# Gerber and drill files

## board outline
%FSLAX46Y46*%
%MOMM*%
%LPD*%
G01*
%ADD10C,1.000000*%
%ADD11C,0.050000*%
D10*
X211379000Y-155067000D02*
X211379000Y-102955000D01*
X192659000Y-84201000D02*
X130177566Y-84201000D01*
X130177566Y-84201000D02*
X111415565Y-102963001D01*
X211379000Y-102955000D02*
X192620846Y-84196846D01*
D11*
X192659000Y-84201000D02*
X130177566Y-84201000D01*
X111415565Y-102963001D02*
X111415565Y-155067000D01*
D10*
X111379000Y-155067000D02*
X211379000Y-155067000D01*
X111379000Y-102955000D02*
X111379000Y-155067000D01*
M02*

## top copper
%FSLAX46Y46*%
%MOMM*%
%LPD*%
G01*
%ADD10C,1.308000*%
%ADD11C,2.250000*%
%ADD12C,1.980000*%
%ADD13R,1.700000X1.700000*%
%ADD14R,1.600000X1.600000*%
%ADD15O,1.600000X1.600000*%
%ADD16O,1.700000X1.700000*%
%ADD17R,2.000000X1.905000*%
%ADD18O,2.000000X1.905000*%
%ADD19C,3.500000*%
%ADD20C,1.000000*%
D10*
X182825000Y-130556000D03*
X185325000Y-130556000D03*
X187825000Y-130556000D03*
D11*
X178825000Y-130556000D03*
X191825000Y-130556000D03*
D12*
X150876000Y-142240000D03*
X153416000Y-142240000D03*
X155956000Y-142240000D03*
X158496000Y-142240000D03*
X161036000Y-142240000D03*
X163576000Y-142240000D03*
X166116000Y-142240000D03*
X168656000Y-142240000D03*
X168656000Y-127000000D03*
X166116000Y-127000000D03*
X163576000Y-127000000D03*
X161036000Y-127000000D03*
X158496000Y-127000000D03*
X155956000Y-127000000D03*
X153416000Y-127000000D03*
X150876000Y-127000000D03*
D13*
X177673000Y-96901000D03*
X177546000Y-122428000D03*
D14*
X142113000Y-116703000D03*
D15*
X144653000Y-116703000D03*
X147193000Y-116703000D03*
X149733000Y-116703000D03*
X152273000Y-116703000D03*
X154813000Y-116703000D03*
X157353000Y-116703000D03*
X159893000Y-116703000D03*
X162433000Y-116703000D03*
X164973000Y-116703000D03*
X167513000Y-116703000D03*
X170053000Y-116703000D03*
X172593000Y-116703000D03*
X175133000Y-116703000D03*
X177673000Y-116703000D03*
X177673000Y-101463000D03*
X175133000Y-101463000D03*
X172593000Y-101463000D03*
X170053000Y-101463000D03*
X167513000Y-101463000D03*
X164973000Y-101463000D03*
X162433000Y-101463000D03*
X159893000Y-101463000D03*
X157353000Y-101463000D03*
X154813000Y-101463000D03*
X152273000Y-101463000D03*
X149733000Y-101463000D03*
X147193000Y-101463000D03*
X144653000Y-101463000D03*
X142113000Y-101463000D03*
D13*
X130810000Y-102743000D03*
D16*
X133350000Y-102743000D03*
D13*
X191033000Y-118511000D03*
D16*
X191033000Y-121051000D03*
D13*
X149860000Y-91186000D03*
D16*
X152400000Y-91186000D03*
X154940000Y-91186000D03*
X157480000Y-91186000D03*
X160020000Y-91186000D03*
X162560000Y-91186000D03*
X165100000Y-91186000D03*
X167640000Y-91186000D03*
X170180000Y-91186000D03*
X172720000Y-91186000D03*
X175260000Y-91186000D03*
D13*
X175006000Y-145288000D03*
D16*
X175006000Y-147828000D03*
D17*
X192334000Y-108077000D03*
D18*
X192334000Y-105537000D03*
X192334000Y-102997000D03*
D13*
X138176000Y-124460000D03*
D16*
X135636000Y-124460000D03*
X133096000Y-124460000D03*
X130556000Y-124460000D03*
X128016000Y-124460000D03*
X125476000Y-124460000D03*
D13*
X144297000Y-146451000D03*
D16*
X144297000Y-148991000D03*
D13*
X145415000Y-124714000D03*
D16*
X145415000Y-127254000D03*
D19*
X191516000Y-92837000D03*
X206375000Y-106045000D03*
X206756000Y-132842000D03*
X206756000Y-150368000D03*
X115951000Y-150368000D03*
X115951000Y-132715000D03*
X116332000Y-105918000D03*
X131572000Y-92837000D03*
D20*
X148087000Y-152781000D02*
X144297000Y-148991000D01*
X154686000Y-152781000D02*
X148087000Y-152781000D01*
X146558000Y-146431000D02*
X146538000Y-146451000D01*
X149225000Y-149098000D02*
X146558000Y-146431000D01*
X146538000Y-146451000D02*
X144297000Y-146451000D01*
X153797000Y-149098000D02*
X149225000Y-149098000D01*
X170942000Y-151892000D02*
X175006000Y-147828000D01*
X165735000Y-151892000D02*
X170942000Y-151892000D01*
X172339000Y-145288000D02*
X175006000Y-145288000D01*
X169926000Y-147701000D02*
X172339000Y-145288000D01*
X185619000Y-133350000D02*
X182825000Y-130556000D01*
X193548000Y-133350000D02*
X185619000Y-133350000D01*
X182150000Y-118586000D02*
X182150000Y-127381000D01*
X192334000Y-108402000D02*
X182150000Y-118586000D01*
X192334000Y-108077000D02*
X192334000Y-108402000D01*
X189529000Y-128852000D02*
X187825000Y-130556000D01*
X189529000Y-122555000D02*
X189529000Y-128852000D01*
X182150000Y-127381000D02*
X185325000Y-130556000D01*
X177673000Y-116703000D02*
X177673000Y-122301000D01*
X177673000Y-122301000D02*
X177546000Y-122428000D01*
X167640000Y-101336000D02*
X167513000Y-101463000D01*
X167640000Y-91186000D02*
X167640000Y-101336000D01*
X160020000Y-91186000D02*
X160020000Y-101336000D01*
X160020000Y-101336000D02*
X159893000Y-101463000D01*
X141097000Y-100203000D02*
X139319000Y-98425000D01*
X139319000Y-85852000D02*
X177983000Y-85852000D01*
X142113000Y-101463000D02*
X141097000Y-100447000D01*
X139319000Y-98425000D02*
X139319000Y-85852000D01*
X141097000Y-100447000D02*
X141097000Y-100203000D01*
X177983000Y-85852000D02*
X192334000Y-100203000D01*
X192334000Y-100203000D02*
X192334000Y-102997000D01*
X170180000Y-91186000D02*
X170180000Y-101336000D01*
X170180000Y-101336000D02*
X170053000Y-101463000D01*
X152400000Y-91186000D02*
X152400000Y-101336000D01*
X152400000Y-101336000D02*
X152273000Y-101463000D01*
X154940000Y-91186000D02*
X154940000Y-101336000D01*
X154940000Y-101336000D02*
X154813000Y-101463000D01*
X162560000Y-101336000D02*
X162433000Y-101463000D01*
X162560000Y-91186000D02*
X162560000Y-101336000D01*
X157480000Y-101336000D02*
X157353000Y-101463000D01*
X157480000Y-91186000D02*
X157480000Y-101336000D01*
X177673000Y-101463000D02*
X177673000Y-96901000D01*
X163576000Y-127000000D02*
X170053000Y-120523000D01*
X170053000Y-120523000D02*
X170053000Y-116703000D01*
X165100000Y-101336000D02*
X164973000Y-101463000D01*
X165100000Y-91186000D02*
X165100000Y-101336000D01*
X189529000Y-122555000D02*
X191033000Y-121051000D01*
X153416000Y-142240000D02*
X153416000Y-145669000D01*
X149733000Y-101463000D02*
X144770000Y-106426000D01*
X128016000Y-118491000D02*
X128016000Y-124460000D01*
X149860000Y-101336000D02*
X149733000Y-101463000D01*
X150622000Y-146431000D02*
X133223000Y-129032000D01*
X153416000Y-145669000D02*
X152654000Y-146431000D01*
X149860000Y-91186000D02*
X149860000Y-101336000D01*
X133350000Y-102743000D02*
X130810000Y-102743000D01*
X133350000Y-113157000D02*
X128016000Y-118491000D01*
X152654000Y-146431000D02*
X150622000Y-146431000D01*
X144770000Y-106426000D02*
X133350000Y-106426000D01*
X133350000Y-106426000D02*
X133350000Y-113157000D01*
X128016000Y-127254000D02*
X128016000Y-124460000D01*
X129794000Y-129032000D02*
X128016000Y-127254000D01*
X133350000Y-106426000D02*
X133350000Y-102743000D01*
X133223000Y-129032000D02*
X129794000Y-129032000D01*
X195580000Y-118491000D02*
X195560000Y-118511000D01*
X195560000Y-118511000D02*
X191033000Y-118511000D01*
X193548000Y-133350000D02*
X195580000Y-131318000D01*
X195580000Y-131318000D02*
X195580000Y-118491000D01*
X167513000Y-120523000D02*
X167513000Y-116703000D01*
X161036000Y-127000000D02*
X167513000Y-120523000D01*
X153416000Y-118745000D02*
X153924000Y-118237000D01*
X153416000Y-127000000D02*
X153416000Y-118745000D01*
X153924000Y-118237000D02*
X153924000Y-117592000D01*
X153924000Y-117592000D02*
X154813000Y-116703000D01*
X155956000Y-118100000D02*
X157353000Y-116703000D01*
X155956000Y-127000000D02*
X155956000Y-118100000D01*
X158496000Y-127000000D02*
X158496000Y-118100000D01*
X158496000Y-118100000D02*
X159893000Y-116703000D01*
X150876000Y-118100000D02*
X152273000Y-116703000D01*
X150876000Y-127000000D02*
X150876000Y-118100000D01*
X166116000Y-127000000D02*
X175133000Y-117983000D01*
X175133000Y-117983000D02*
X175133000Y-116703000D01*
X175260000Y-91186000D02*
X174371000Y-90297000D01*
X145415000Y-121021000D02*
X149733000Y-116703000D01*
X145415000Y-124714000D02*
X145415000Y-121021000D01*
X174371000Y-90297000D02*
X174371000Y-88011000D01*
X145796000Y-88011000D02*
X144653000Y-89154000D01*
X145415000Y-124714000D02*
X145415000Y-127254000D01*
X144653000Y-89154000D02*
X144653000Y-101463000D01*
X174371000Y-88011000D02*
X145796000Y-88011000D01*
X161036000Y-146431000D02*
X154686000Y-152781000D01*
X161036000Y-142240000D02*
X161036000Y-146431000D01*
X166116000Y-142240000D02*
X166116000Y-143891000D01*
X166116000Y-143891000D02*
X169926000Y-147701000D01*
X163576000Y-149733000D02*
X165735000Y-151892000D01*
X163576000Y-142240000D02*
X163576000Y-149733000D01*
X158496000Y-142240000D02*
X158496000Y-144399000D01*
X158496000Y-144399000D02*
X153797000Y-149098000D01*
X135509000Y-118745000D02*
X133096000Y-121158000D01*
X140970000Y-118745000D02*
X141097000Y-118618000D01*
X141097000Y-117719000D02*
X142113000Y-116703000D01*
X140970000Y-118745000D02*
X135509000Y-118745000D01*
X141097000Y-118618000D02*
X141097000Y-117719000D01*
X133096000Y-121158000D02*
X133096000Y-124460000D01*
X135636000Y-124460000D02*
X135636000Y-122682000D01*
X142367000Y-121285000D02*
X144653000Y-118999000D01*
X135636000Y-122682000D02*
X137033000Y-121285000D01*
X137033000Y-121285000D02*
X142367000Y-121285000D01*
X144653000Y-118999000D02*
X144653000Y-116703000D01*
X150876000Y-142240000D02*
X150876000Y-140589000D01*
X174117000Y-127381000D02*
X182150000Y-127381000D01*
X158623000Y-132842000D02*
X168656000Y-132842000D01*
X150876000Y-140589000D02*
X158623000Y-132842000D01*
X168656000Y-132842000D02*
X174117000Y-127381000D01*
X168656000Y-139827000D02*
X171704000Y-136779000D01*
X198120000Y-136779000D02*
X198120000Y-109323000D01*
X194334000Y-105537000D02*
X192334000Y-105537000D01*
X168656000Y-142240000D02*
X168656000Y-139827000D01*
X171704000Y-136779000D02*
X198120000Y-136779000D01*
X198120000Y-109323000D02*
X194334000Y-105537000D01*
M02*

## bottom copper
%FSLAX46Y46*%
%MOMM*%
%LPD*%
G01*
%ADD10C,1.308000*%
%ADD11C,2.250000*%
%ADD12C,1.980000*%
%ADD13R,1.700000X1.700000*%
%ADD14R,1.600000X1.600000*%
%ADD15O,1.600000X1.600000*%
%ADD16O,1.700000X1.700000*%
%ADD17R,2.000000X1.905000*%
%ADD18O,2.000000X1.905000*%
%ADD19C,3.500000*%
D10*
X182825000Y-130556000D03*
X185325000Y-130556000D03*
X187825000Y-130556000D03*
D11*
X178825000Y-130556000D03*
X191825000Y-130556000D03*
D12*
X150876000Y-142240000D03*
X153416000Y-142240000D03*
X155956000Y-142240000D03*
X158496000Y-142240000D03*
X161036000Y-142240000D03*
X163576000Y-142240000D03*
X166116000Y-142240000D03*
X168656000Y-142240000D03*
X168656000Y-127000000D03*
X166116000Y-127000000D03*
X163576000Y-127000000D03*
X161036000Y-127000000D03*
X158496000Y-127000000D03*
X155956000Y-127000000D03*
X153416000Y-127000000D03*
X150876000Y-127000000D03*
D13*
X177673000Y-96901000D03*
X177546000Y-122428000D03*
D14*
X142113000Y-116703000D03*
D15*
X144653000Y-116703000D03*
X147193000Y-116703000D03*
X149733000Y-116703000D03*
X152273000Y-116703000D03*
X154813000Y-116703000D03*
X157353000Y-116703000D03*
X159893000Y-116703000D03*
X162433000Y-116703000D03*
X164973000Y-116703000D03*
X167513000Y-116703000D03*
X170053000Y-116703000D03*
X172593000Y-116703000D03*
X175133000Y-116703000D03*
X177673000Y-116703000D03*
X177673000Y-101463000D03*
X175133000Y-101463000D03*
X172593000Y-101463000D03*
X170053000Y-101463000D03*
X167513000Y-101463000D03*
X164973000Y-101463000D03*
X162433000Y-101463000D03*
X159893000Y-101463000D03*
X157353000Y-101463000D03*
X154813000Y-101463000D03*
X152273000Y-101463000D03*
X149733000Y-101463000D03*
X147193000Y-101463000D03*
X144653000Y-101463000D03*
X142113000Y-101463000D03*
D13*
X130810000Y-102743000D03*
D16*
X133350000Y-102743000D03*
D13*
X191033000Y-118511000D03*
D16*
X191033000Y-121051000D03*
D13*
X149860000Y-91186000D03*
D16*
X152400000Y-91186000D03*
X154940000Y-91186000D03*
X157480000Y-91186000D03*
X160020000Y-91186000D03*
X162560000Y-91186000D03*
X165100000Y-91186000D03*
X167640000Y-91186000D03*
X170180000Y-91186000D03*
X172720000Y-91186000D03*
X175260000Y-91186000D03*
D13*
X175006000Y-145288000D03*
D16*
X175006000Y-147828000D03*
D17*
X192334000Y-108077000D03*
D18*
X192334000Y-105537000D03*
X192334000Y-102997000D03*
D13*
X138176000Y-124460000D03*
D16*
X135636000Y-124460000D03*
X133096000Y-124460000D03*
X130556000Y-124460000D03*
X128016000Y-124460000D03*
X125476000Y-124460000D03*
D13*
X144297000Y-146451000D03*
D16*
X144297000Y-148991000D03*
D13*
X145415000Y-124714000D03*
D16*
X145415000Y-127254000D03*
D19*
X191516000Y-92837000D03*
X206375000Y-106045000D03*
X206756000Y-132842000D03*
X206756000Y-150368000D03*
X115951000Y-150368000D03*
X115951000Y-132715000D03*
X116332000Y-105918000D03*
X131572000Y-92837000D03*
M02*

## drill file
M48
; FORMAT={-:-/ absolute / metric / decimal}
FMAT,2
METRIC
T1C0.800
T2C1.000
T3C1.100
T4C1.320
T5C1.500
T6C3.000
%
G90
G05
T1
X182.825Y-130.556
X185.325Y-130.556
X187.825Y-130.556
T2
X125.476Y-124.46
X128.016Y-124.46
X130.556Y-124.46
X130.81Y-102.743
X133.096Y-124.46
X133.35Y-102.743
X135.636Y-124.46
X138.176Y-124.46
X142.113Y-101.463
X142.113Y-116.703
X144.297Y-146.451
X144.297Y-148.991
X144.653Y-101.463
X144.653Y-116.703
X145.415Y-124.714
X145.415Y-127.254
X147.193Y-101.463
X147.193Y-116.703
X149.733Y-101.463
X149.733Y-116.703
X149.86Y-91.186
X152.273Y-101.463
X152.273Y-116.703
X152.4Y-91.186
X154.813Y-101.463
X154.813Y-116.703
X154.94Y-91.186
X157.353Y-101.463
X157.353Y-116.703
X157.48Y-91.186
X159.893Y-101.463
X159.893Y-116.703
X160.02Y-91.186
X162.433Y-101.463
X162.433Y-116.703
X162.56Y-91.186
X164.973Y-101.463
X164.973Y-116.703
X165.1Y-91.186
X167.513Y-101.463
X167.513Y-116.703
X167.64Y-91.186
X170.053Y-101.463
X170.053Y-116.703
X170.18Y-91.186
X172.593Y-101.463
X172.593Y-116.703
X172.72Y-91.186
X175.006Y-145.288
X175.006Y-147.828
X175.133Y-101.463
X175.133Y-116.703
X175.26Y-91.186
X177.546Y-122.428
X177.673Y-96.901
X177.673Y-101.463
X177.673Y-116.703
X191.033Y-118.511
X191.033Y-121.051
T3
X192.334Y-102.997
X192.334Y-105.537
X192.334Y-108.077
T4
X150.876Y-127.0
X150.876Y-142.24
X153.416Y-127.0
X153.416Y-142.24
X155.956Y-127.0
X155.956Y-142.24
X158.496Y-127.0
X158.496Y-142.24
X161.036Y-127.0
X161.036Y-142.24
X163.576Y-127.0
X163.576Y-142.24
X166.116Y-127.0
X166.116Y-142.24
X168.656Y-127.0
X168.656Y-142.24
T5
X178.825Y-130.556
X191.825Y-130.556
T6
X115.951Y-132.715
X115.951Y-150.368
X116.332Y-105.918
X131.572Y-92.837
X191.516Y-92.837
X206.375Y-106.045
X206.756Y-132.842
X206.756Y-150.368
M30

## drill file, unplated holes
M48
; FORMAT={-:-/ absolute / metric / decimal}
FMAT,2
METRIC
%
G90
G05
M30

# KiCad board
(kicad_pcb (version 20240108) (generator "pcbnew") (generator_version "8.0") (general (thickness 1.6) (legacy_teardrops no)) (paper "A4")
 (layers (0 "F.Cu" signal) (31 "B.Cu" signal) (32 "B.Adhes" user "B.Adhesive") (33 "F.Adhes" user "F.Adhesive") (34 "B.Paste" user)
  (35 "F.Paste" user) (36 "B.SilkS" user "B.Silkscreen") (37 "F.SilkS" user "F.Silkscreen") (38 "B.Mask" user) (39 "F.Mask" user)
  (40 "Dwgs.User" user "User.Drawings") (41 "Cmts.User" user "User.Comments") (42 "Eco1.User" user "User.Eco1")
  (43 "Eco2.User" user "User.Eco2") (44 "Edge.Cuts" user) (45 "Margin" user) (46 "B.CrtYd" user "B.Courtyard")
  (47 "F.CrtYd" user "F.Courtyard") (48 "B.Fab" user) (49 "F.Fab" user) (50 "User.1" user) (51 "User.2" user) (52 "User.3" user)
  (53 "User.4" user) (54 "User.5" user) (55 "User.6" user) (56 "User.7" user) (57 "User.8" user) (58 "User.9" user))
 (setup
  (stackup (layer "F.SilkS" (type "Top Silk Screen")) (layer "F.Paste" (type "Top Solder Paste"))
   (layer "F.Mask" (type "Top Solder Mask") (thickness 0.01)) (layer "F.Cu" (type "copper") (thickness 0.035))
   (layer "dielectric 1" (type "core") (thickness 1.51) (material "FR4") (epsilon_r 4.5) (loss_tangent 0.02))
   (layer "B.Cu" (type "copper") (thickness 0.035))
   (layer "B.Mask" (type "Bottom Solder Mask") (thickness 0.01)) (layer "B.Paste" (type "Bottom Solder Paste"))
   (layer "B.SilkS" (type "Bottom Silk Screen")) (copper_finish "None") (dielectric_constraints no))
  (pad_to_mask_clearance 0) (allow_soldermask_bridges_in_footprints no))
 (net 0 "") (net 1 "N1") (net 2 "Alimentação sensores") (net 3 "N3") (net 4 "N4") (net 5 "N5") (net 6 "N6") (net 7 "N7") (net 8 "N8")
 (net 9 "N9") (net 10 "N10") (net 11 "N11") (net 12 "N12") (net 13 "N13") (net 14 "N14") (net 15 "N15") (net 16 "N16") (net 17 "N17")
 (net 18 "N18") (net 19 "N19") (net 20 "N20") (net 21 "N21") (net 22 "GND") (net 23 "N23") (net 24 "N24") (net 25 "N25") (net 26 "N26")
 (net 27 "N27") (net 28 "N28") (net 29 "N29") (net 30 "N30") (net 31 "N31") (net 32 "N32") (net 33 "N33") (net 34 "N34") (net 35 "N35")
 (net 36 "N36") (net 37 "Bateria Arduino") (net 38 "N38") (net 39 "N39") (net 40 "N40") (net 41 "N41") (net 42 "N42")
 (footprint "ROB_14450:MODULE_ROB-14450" (layer "F.Cu") (at 159.766 134.62 90)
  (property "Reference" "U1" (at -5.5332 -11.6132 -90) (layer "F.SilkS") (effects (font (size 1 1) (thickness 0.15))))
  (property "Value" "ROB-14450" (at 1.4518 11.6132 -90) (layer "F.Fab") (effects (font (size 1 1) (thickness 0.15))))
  (pad "1" thru_hole circle (at -7.62 -8.89 90) (size 1.98 1.98) (drill 1.32) (layers "*.Cu" "*.Mask") (remove_unused_layers no)
   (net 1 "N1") (solder_mask_margin 0.102))
  (pad "2" thru_hole circle (at -7.62 -6.35 90) (size 1.98 1.98) (drill 1.32) (layers "*.Cu" "*.Mask") (remove_unused_layers no)
   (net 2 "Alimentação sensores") (solder_mask_margin 0.102))
  (pad "3" thru_hole circle (at -7.62 -3.81 90) (size 1.98 1.98) (drill 1.32) (layers "*.Cu" "*.Mask") (remove_unused_layers no)
   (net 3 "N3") (solder_mask_margin 0.102))
  (pad "4" thru_hole circle (at -7.62 -1.27 90) (size 1.98 1.98) (drill 1.32) (layers "*.Cu" "*.Mask") (remove_unused_layers no)
   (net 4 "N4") (solder_mask_margin 0.102))
  (pad "5" thru_hole circle (at -7.62 1.27 90) (size 1.98 1.98) (drill 1.32) (layers "*.Cu" "*.Mask") (remove_unused_layers no) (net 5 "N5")
   (solder_mask_margin 0.102))
  (pad "6" thru_hole circle (at -7.62 3.81 90) (size 1.98 1.98) (drill 1.32) (layers "*.Cu" "*.Mask") (remove_unused_layers no) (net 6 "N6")
   (solder_mask_margin 0.102))
  (pad "7" thru_hole circle (at -7.62 6.35 90) (size 1.98 1.98) (drill 1.32) (layers "*.Cu" "*.Mask") (remove_unused_layers no) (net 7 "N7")
   (solder_mask_margin 0.102))
  (pad "8" thru_hole circle (at -7.62 8.89 90) (size 1.98 1.98) (drill 1.32) (layers "*.Cu" "*.Mask") (remove_unused_layers no) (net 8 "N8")
   (solder_mask_margin 0.102))
  (pad "9" thru_hole circle (at 7.62 8.89 90) (size 1.98 1.98) (drill 1.32) (layers "*.Cu" "*.Mask") (remove_unused_layers no) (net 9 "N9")
   (solder_mask_margin 0.102))
  (pad "10" thru_hole circle (at 7.62 6.35 90) (size 1.98 1.98) (drill 1.32) (layers "*.Cu" "*.Mask") (remove_unused_layers no)
   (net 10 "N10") (solder_mask_margin 0.102))
  (pad "11" thru_hole circle (at 7.62 3.81 90) (size 1.98 1.98) (drill 1.32) (layers "*.Cu" "*.Mask") (remove_unused_layers no)
   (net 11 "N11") (solder_mask_margin 0.102))
  (pad "12" thru_hole circle (at 7.62 1.27 90) (size 1.98 1.98) (drill 1.32) (layers "*.Cu" "*.Mask") (remove_unused_layers no)
   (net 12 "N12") (solder_mask_margin 0.102))
  (pad "13" thru_hole circle (at 7.62 -1.27 90) (size 1.98 1.98) (drill 1.32) (layers "*.Cu" "*.Mask") (remove_unused_layers no)
   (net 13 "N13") (solder_mask_margin 0.102))
  (pad "14" thru_hole circle (at 7.62 -3.81 90) (size 1.98 1.98) (drill 1.32) (layers "*.Cu" "*.Mask") (remove_unused_layers no)
   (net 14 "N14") (solder_mask_margin 0.102))
  (pad "15" thru_hole circle (at 7.62 -6.35 90) (size 1.98 1.98) (drill 1.32) (layers "*.Cu" "*.Mask") (remove_unused_layers no)
   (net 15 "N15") (solder_mask_margin 0.102))
  (pad "16" thru_hole circle (at 7.62 -8.89 90) (size 1.98 1.98) (drill 1.32) (layers "*.Cu" "*.Mask") (remove_unused_layers no)
   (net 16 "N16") (solder_mask_margin 0.102)))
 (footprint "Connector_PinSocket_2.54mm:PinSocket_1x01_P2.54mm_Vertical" (layer "F.Cu") (at 177.673 96.901)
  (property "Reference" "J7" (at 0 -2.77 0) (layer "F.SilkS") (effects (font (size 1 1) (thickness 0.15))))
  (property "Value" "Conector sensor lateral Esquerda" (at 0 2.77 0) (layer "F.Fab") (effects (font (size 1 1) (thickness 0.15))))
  (pad "1" thru_hole rect (at 0 0) (size 1.7 1.7) (drill 1) (layers "*.Cu" "*.Mask") (remove_unused_layers no) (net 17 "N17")))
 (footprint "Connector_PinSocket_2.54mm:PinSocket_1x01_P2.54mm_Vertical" (layer "F.Cu") (at 177.546 122.428)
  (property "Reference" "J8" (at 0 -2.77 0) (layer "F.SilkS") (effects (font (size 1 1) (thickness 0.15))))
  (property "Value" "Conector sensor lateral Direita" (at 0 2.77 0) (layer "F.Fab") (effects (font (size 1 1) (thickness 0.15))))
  (pad "1" thru_hole rect (at 0 0) (size 1.7 1.7) (drill 1) (layers "*.Cu" "*.Mask") (remove_unused_layers no) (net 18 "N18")))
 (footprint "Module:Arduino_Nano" (layer "F.Cu") (at 142.113 116.703 90)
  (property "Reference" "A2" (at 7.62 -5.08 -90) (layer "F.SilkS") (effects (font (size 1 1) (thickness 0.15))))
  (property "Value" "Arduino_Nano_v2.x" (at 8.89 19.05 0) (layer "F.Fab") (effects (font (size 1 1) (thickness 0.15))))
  (pad "1" thru_hole rect (at 0 0 90) (size 1.6 1.6) (drill 1) (layers "*.Cu" "*.Mask") (remove_unused_layers no) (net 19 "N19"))
  (pad "2" thru_hole oval (at 0 2.54 90) (size 1.6 1.6) (drill 1) (layers "*.Cu" "*.Mask") (remove_unused_layers no) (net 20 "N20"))
  (pad "3" thru_hole oval (at 0 5.08 90) (size 1.6 1.6) (drill 1) (layers "*.Cu" "*.Mask") (remove_unused_layers no) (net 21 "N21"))
  (pad "4" thru_hole oval (at 0 7.62 90) (size 1.6 1.6) (drill 1) (layers "*.Cu" "*.Mask") (remove_unused_layers no) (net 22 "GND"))
  (pad "5" thru_hole oval (at 0 10.16 90) (size 1.6 1.6) (drill 1) (layers "*.Cu" "*.Mask") (remove_unused_layers no) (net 16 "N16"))
  (pad "6" thru_hole oval (at 0 12.7 90) (size 1.6 1.6) (drill 1) (layers "*.Cu" "*.Mask") (remove_unused_layers no) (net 15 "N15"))
  (pad "7" thru_hole oval (at 0 15.24 90) (size 1.6 1.6) (drill 1) (layers "*.Cu" "*.Mask") (remove_unused_layers no) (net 14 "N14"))
  (pad "8" thru_hole oval (at 0 17.78 90) (size 1.6 1.6) (drill 1) (layers "*.Cu" "*.Mask") (remove_unused_layers no) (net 13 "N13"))
  (pad "9" thru_hole oval (at 0 20.32 90) (size 1.6 1.6) (drill 1) (layers "*.Cu" "*.Mask") (remove_unused_layers no) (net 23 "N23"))
  (pad "10" thru_hole oval (at 0 22.86 90) (size 1.6 1.6) (drill 1) (layers "*.Cu" "*.Mask") (remove_unused_layers no) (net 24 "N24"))
  (pad "11" thru_hole oval (at 0 25.4 90) (size 1.6 1.6) (drill 1) (layers "*.Cu" "*.Mask") (remove_unused_layers no) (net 12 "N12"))
  (pad "12" thru_hole oval (at 0 27.94 90) (size 1.6 1.6) (drill 1) (layers "*.Cu" "*.Mask") (remove_unused_layers no) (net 11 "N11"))
  (pad "13" thru_hole oval (at 0 30.48 90) (size 1.6 1.6) (drill 1) (layers "*.Cu" "*.Mask") (remove_unused_layers no) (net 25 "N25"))
  (pad "14" thru_hole oval (at 0 33.02 90) (size 1.6 1.6) (drill 1) (layers "*.Cu" "*.Mask") (remove_unused_layers no) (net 10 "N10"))
  (pad "15" thru_hole oval (at 0 35.56 90) (size 1.6 1.6) (drill 1) (layers "*.Cu" "*.Mask") (remove_unused_layers no) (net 18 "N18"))
  (pad "16" thru_hole oval (at 15.24 35.56 90) (size 1.6 1.6) (drill 1) (layers "*.Cu" "*.Mask") (remove_unused_layers no) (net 17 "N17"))
  (pad "17" thru_hole oval (at 15.24 33.02 90) (size 1.6 1.6) (drill 1) (layers "*.Cu" "*.Mask") (remove_unused_layers no) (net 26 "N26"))
  (pad "18" thru_hole oval (at 15.24 30.48 90) (size 1.6 1.6) (drill 1) (layers "*.Cu" "*.Mask") (remove_unused_layers no) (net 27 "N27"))
  (pad "19" thru_hole oval (at 15.24 27.94 90) (size 1.6 1.6) (drill 1) (layers "*.Cu" "*.Mask") (remove_unused_layers no) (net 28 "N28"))
  (pad "20" thru_hole oval (at 15.24 25.4 90) (size 1.6 1.6) (drill 1) (layers "*.Cu" "*.Mask") (remove_unused_layers no) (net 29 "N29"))
  (pad "21" thru_hole oval (at 15.24 22.86 90) (size 1.6 1.6) (drill 1) (layers "*.Cu" "*.Mask") (remove_unused_layers no) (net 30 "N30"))
  (pad "22" thru_hole oval (at 15.24 20.32 90) (size 1.6 1.6) (drill 1) (layers "*.Cu" "*.Mask") (remove_unused_layers no) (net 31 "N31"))
  (pad "23" thru_hole oval (at 15.24 17.78 90) (size 1.6 1.6) (drill 1) (layers "*.Cu" "*.Mask") (remove_unused_layers no) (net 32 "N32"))
  (pad "24" thru_hole oval (at 15.24 15.24 90) (size 1.6 1.6) (drill 1) (layers "*.Cu" "*.Mask") (remove_unused_layers no) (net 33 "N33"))
  (pad "25" thru_hole oval (at 15.24 12.7 90) (size 1.6 1.6) (drill 1) (layers "*.Cu" "*.Mask") (remove_unused_layers no) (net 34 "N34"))
  (pad "26" thru_hole oval (at 15.24 10.16 90) (size 1.6 1.6) (drill 1) (layers "*.Cu" "*.Mask") (remove_unused_layers no) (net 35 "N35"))
  (pad "27" thru_hole oval (at 15.24 7.62 90) (size 1.6 1.6) (drill 1) (layers "*.Cu" "*.Mask") (remove_unused_layers no)
   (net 2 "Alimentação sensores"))
  (pad "28" thru_hole oval (at 15.24 5.08 90) (size 1.6 1.6) (drill 1) (layers "*.Cu" "*.Mask") (remove_unused_layers no) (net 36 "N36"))
  (pad "29" thru_hole oval (at 15.24 2.54 90) (size 1.6 1.6) (drill 1) (layers "*.Cu" "*.Mask") (remove_unused_layers no) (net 22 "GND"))
  (pad "30" thru_hole oval (at 15.24 0 90) (size 1.6 1.6) (drill 1) (layers "*.Cu" "*.Mask") (remove_unused_layers no)
   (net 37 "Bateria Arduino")))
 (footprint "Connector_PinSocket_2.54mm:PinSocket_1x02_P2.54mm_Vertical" (layer "F.Cu") (at 130.81 102.743 90)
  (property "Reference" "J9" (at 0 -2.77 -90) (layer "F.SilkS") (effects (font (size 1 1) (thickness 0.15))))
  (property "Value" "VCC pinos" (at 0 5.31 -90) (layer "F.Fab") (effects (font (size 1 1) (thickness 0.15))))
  (pad "1" thru_hole rect (at 0 0 90) (size 1.7 1.7) (drill 1) (layers "*.Cu" "*.Mask") (remove_unused_layers no)
   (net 2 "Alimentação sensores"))
  (pad "2" thru_hole oval (at 0 2.54 90) (size 1.7 1.7) (drill 1) (layers "*.Cu" "*.Mask") (remove_unused_layers no)
   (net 2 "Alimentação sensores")))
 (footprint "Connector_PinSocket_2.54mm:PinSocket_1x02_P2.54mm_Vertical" (layer "F.Cu") (at 191.033 118.511)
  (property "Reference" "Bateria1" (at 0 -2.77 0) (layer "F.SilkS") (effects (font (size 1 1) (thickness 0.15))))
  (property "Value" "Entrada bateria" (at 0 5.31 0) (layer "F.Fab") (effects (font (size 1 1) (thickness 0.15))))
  (pad "1" thru_hole rect (at 0 0) (size 1.7 1.7) (drill 1) (layers "*.Cu" "*.Mask") (remove_unused_layers no) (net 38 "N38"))
  (pad "2" thru_hole oval (at 0 2.54) (size 1.7 1.7) (drill 1) (layers "*.Cu" "*.Mask") (remove_unused_layers no) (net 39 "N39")))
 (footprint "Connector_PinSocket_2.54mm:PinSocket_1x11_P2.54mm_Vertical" (layer "F.Cu") (at 149.86 91.186 90)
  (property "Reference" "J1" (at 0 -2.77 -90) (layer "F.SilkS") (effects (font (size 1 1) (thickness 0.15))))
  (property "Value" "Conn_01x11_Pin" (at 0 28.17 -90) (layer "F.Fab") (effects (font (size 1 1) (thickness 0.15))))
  (pad "1" thru_hole rect (at 0 0 90) (size 1.7 1.7) (drill 1) (layers "*.Cu" "*.Mask") (remove_unused_layers no)
   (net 2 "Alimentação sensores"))
  (pad "2" thru_hole oval (at 0 2.54 90) (size 1.7 1.7) (drill 1) (layers "*.Cu" "*.Mask") (remove_unused_layers no) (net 35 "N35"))
  (pad "3" thru_hole oval (at 0 5.08 90) (size 1.7 1.7) (drill 1) (layers "*.Cu" "*.Mask") (remove_unused_layers no) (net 34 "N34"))
  (pad "4" thru_hole oval (at 0 7.62 90) (size 1.7 1.7) (drill 1) (layers "*.Cu" "*.Mask") (remove_unused_layers no) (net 33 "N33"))
  (pad "5" thru_hole oval (at 0 10.16 90) (size 1.7 1.7) (drill 1) (layers "*.Cu" "*.Mask") (remove_unused_layers no) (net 32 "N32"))
  (pad "6" thru_hole oval (at 0 12.7 90) (size 1.7 1.7) (drill 1) (layers "*.Cu" "*.Mask") (remove_unused_layers no) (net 31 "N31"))
  (pad "7" thru_hole oval (at 0 15.24 90) (size 1.7 1.7) (drill 1) (layers "*.Cu" "*.Mask") (remove_unused_layers no) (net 30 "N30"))
  (pad "8" thru_hole oval (at 0 17.78 90) (size 1.7 1.7) (drill 1) (layers "*.Cu" "*.Mask") (remove_unused_layers no) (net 29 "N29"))
  (pad "9" thru_hole oval (at 0 20.32 90) (size 1.7 1.7) (drill 1) (layers "*.Cu" "*.Mask") (remove_unused_layers no) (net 28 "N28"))
  (pad "10" thru_hole oval (at 0 22.86 90) (size 1.7 1.7) (drill 1) (layers "*.Cu" "*.Mask") (remove_unused_layers no) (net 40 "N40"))
  (pad "11" thru_hole oval (at 0 25.4 90) (size 1.7 1.7) (drill 1) (layers "*.Cu" "*.Mask") (remove_unused_layers no) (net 22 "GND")))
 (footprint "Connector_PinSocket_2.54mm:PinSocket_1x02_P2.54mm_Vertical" (layer "F.Cu") (at 175.006 145.288)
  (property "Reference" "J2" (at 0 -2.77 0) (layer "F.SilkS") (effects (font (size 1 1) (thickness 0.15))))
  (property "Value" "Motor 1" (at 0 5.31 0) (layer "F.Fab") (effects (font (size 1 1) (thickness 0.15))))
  (pad "1" thru_hole rect (at 0 0) (size 1.7 1.7) (drill 1) (layers "*.Cu" "*.Mask") (remove_unused_layers no) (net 7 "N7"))
  (pad "2" thru_hole oval (at 0 2.54) (size 1.7 1.7) (drill 1) (layers "*.Cu" "*.Mask") (remove_unused_layers no) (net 6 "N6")))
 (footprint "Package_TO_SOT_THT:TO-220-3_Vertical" (layer "F.Cu") (at 192.334 108.077 90)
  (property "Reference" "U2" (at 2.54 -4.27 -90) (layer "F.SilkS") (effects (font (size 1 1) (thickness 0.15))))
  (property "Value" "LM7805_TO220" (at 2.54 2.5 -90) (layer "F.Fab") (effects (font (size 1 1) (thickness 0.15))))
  (pad "1" thru_hole rect (at 0 0 90) (size 1.905 2) (drill 1.1) (layers "*.Cu" "*.Mask") (remove_unused_layers no) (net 1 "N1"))
  (pad "2" thru_hole oval (at 2.54 0 90) (size 1.905 2) (drill 1.1) (layers "*.Cu" "*.Mask") (remove_unused_layers no) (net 8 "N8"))
  (pad "3" thru_hole oval (at 5.08 0 90) (size 1.905 2) (drill 1.1) (layers "*.Cu" "*.Mask") (remove_unused_layers no)
   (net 37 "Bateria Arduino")))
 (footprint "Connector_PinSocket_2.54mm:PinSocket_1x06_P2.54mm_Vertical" (layer "F.Cu") (at 138.176 124.46 -90)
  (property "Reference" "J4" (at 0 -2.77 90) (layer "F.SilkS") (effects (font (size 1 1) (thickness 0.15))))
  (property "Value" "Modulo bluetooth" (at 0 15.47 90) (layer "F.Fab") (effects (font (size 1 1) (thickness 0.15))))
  (pad "1" thru_hole rect (at 0 0 270) (size 1.7 1.7) (drill 1) (layers "*.Cu" "*.Mask") (remove_unused_layers no) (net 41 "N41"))
  (pad "2" thru_hole oval (at 0 2.54 270) (size 1.7 1.7) (drill 1) (layers "*.Cu" "*.Mask") (remove_unused_layers no) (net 20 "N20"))
  (pad "3" thru_hole oval (at 0 5.08 270) (size 1.7 1.7) (drill 1) (layers "*.Cu" "*.Mask") (remove_unused_layers no) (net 19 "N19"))
  (pad "4" thru_hole oval (at 0 7.62 270) (size 1.7 1.7) (drill 1) (layers "*.Cu" "*.Mask") (remove_unused_layers no) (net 22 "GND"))
  (pad "5" thru_hole oval (at 0 10.16 270) (size 1.7 1.7) (drill 1) (layers "*.Cu" "*.Mask") (remove_unused_layers no)
   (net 2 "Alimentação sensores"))
  (pad "6" thru_hole oval (at 0 12.7 270) (size 1.7 1.7) (drill 1) (layers "*.Cu" "*.Mask") (remove_unused_layers no) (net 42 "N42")))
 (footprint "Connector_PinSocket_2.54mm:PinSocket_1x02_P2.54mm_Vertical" (layer "F.Cu") (at 144.297 146.451)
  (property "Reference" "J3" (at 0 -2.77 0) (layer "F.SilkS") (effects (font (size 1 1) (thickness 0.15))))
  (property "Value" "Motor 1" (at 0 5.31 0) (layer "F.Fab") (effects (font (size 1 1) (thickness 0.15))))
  (pad "1" thru_hole rect (at 0 0) (size 1.7 1.7) (drill 1) (layers "*.Cu" "*.Mask") (remove_unused_layers no) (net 4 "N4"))
  (pad "2" thru_hole oval (at 0 2.54) (size 1.7 1.7) (drill 1) (layers "*.Cu" "*.Mask") (remove_unused_layers no) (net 5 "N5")))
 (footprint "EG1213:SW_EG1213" (layer "F.Cu") (at 185.325 130.556)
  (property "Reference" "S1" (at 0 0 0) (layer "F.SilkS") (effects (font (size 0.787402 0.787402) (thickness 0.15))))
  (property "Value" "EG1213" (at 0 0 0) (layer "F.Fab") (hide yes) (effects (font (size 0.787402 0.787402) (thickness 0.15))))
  (pad "1" thru_hole circle (at -2.5 0) (size 1.308 1.308) (drill 0.8) (layers "*.Cu" "*.Mask") (remove_unused_layers no) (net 38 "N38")
   (solder_mask_margin 0.102))
  (pad "2" thru_hole circle (at 0 0) (size 1.308 1.308) (drill 0.8) (layers "*.Cu" "*.Mask") (remove_unused_layers no) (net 1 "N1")
   (solder_mask_margin 0.102))
  (pad "3" thru_hole circle (at 2.5 0) (size 1.308 1.308) (drill 0.8) (layers "*.Cu" "*.Mask") (remove_unused_layers no) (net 39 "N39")
   (solder_mask_margin 0.102))
  (pad "P$4" thru_hole circle (at -6.5 0) (size 2.25 2.25) (drill 1.5) (layers "*.Cu" "*.Mask") (remove_unused_layers no)
   (solder_mask_margin 0.102))
  (pad "P$5" thru_hole circle (at 6.5 0) (size 2.25 2.25) (drill 1.5) (layers "*.Cu" "*.Mask") (remove_unused_layers no)
   (solder_mask_margin 0.102)))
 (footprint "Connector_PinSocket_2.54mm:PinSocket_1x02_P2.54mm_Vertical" (layer "F.Cu") (at 145.415 124.714)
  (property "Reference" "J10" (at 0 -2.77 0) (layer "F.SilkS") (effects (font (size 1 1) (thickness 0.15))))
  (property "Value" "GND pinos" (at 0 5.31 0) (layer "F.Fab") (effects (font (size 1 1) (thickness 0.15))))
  (pad "1" thru_hole rect (at 0 0) (size 1.7 1.7) (drill 1) (layers "*.Cu" "*.Mask") (remove_unused_layers no) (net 22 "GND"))
  (pad "2" thru_hole oval (at 0 2.54) (size 1.7 1.7) (drill 1) (layers "*.Cu" "*.Mask") (remove_unused_layers no) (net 22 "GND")))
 (gr_line (start 211.379 155.067) (end 211.379 102.955) (stroke (width 1) (type default)) (layer "Edge.Cuts"))
 (gr_line (start 192.659 84.201) (end 130.177566 84.201) (stroke (width 1) (type default)) (layer "Edge.Cuts"))
 (gr_line (start 130.177566 84.201) (end 111.415565 102.963001) (stroke (width 1) (type default)) (layer "Edge.Cuts"))
 (gr_line (start 211.379 102.955) (end 192.620846 84.196846) (stroke (width 1) (type default)) (layer "Edge.Cuts"))
 (gr_line (start 192.659 84.201) (end 130.177566 84.201) (stroke (width 0.05) (type default)) (layer "Edge.Cuts"))
 (gr_line (start 111.415565 102.963001) (end 111.415565 155.067) (stroke (width 0.05) (type default)) (layer "Edge.Cuts"))
 (gr_line (start 111.379 155.067) (end 211.379 155.067) (stroke (width 1) (type default)) (layer "Edge.Cuts"))
 (gr_line (start 111.379 102.955) (end 111.379 155.067) (stroke (width 1) (type default)) (layer "Edge.Cuts"))
 (via (at 116.332 105.918) (size 3.5) (drill 3) (layers "F.Cu" "B.Cu") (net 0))
 (via (at 206.756 150.368) (size 3.5) (drill 3) (layers "F.Cu" "B.Cu") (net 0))
 (via (at 191.516 92.837) (size 3.5) (drill 3) (layers "F.Cu" "B.Cu") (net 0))
 (via (at 131.572 92.837) (size 3.5) (drill 3) (layers "F.Cu" "B.Cu") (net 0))
 (via (at 206.756 132.842) (size 3.5) (drill 3) (layers "F.Cu" "B.Cu") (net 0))
 (via (at 206.375 106.045) (size 3.5) (drill 3) (layers "F.Cu" "B.Cu") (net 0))
 (via (at 115.951 132.715) (size 3.5) (drill 3) (layers "F.Cu" "B.Cu") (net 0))
 (via (at 115.951 150.368) (size 3.5) (drill 3) (layers "F.Cu" "B.Cu") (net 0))
 (segment (start 177.673 116.703) (end 177.673 122.301) (width 1) (layer "F.Cu") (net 18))
 (segment (start 177.673 122.301) (end 177.546 122.428) (width 1) (layer "F.Cu") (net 18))
 (segment (start 167.64 101.336) (end 167.513 101.463) (width 1) (layer "F.Cu") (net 29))
 (segment (start 167.64 91.186) (end 167.64 101.336) (width 1) (layer "F.Cu") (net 29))
 (segment (start 160.02 91.186) (end 160.02 101.336) (width 1) (layer "F.Cu") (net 32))
 (segment (start 160.02 101.336) (end 159.893 101.463) (width 1) (layer "F.Cu") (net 32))
 (segment (start 141.097 100.203) (end 139.319 98.425) (width 1) (layer "F.Cu") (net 37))
 (segment (start 139.319 85.852) (end 177.983 85.852) (width 1) (layer "F.Cu") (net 37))
 (segment (start 142.113 101.463) (end 141.097 100.447) (width 1) (layer "F.Cu") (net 37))
 (segment (start 139.319 98.425) (end 139.319 85.852) (width 1) (layer "F.Cu") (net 37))
 (segment (start 141.097 100.447) (end 141.097 100.203) (width 1) (layer "F.Cu") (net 37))
 (segment (start 177.983 85.852) (end 192.334 100.203) (width 1) (layer "F.Cu") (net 37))
 (segment (start 192.334 100.203) (end 192.334 102.997) (width 1) (layer "F.Cu") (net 37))
 (segment (start 170.18 91.186) (end 170.18 101.336) (width 1) (layer "F.Cu") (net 28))
 (segment (start 170.18 101.336) (end 170.053 101.463) (width 1) (layer "F.Cu") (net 28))
 (segment (start 152.4 91.186) (end 152.4 101.336) (width 1) (layer "F.Cu") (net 35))
 (segment (start 152.4 101.336) (end 152.273 101.463) (width 1) (layer "F.Cu") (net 35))
 (segment (start 154.94 91.186) (end 154.94 101.336) (width 1) (layer "F.Cu") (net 34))
 (segment (start 154.94 101.336) (end 154.813 101.463) (width 1) (layer "F.Cu") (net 34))
 (segment (start 162.56 101.336) (end 162.433 101.463) (width 1) (layer "F.Cu") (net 31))
 (segment (start 162.56 91.186) (end 162.56 101.336) (width 1) (layer "F.Cu") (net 31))
 (segment (start 157.48 101.336) (end 157.353 101.463) (width 1) (layer "F.Cu") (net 33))
 (segment (start 157.48 91.186) (end 157.48 101.336) (width 1) (layer "F.Cu") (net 33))
 (segment (start 177.673 101.463) (end 177.673 96.901) (width 1) (layer "F.Cu") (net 17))
 (segment (start 163.576 127) (end 170.053 120.523) (width 1) (layer "F.Cu") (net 11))
 (segment (start 170.053 120.523) (end 170.053 116.703) (width 1) (layer "F.Cu") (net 11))
 (segment (start 165.1 101.336) (end 164.973 101.463) (width 1) (layer "F.Cu") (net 30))
 (segment (start 165.1 91.186) (end 165.1 101.336) (width 1) (layer "F.Cu") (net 30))
 (segment (start 189.529 128.852) (end 187.825 130.556) (width 1) (layer "F.Cu") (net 39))
 (segment (start 189.529 122.555) (end 191.033 121.051) (width 1) (layer "F.Cu") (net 39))
 (segment (start 189.529 122.555) (end 189.529 128.852) (width 1) (layer "F.Cu") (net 39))
 (segment (start 153.416 142.24) (end 153.416 145.669) (width 1) (layer "F.Cu") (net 2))
 (segment (start 149.733 101.463) (end 144.77 106.426) (width 1) (layer "F.Cu") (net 2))
 (segment (start 128.016 118.491) (end 128.016 124.46) (width 1) (layer "F.Cu") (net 2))
 (segment (start 149.86 101.336) (end 149.733 101.463) (width 1) (layer "F.Cu") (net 2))
 (segment (start 150.622 146.431) (end 133.223 129.032) (width 1) (layer "F.Cu") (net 2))
 (segment (start 153.416 145.669) (end 152.654 146.431) (width 1) (layer "F.Cu") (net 2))
 (segment (start 149.86 91.186) (end 149.86 101.336) (width 1) (layer "F.Cu") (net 2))
 (segment (start 133.35 102.743) (end 130.81 102.743) (width 1) (layer "F.Cu") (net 2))
 (segment (start 133.35 113.157) (end 128.016 118.491) (width 1) (layer "F.Cu") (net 2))
 (segment (start 152.654 146.431) (end 150.622 146.431) (width 1) (layer "F.Cu") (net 2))
 (segment (start 144.77 106.426) (end 133.35 106.426) (width 1) (layer "F.Cu") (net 2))
 (segment (start 133.35 106.426) (end 133.35 113.157) (width 1) (layer "F.Cu") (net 2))
 (segment (start 128.016 127.254) (end 128.016 124.46) (width 1) (layer "F.Cu") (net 2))
 (segment (start 129.794 129.032) (end 128.016 127.254) (width 1) (layer "F.Cu") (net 2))
 (segment (start 133.35 106.426) (end 133.35 102.743) (width 1) (layer "F.Cu") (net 2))
 (segment (start 133.223 129.032) (end 129.794 129.032) (width 1) (layer "F.Cu") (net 2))
 (segment (start 195.58 118.491) (end 195.56 118.511) (width 1) (layer "F.Cu") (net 38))
 (segment (start 193.548 133.35) (end 185.619 133.35) (width 1) (layer "F.Cu") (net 38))
 (segment (start 185.619 133.35) (end 182.825 130.556) (width 1) (layer "F.Cu") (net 38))
 (segment (start 195.56 118.511) (end 191.033 118.511) (width 1) (layer "F.Cu") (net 38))
 (segment (start 193.548 133.35) (end 195.58 131.318) (width 1) (layer "F.Cu") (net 38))
 (segment (start 195.58 131.318) (end 195.58 118.491) (width 1) (layer "F.Cu") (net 38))
 (segment (start 167.513 120.523) (end 167.513 116.703) (width 1) (layer "F.Cu") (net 12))
 (segment (start 161.036 127) (end 167.513 120.523) (width 1) (layer "F.Cu") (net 12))
 (segment (start 153.416 118.745) (end 153.924 118.237) (width 1) (layer "F.Cu") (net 15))
 (segment (start 153.416 127) (end 153.416 118.745) (width 1) (layer "F.Cu") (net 15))
 (segment (start 153.924 118.237) (end 153.924 117.592) (width 1) (layer "F.Cu") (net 15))
 (segment (start 153.924 117.592) (end 154.813 116.703) (width 1) (layer "F.Cu") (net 15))
 (segment (start 155.956 118.1) (end 157.353 116.703) (width 1) (layer "F.Cu") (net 14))
 (segment (start 155.956 127) (end 155.956 118.1) (width 1) (layer "F.Cu") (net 14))
 (segment (start 158.496 127) (end 158.496 118.1) (width 1) (layer "F.Cu") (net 13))
 (segment (start 158.496 118.1) (end 159.893 116.703) (width 1) (layer "F.Cu") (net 13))
 (segment (start 150.876 118.1) (end 152.273 116.703) (width 1) (layer "F.Cu") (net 16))
 (segment (start 150.876 127) (end 150.876 118.1) (width 1) (layer "F.Cu") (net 16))
 (segment (start 166.116 127) (end 175.133 117.983) (width 1) (layer "F.Cu") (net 10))
 (segment (start 175.133 117.983) (end 175.133 116.703) (width 1) (layer "F.Cu") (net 10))
 (segment (start 175.26 91.186) (end 174.371 90.297) (width 1) (layer "F.Cu") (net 22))
 (segment (start 145.415 121.021) (end 149.733 116.703) (width 1) (layer "F.Cu") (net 22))
 (segment (start 145.415 124.714) (end 145.415 121.021) (width 1) (layer "F.Cu") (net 22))
 (segment (start 174.371 90.297) (end 174.371 88.011) (width 1) (layer "F.Cu") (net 22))
 (segment (start 145.796 88.011) (end 144.653 89.154) (width 1) (layer "F.Cu") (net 22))
 (segment (start 145.415 124.714) (end 145.415 127.254) (width 1) (layer "F.Cu") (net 22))
 (segment (start 144.653 89.154) (end 144.653 101.463) (width 1) (layer "F.Cu") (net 22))
 (segment (start 174.371 88.011) (end 145.796 88.011) (width 1) (layer "F.Cu") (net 22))
 (segment (start 148.087 152.781) (end 144.297 148.991) (width 1) (layer "F.Cu") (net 5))
 (segment (start 161.036 146.431) (end 154.686 152.781) (width 1) (layer "F.Cu") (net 5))
 (segment (start 154.686 152.781) (end 148.087 152.781) (width 1) (layer "F.Cu") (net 5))
 (segment (start 161.036 142.24) (end 161.036 146.431) (width 1) (layer "F.Cu") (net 5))
 (segment (start 166.116 142.24) (end 166.116 143.891) (width 1) (layer "F.Cu") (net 7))
 (segment (start 169.926 147.701) (end 172.339 145.288) (width 1) (layer "F.Cu") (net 7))
 (segment (start 172.339 145.288) (end 175.006 145.288) (width 1) (layer "F.Cu") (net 7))
 (segment (start 166.116 143.891) (end 169.926 147.701) (width 1) (layer "F.Cu") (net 7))
 (segment (start 170.942 151.892) (end 175.006 147.828) (width 1) (layer "F.Cu") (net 6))
 (segment (start 163.576 149.733) (end 165.735 151.892) (width 1) (layer "F.Cu") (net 6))
 (segment (start 163.576 142.24) (end 163.576 149.733) (width 1) (layer "F.Cu") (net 6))
 (segment (start 165.735 151.892) (end 170.942 151.892) (width 1) (layer "F.Cu") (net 6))
 (segment (start 146.558 146.431) (end 146.538 146.451) (width 1) (layer "F.Cu") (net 4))
 (segment (start 146.538 146.451) (end 144.297 146.451) (width 1) (layer "F.Cu") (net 4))
 (segment (start 149.225 149.098) (end 146.558 146.431) (width 1) (layer "F.Cu") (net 4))
 (segment (start 158.496 142.24) (end 158.496 144.399) (width 1) (layer "F.Cu") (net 4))
 (segment (start 153.797 149.098) (end 149.225 149.098) (width 1) (layer "F.Cu") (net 4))
 (segment (start 158.496 144.399) (end 153.797 149.098) (width 1) (layer "F.Cu") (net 4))
 (segment (start 135.509 118.745) (end 133.096 121.158) (width 1) (layer "F.Cu") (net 19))
 (segment (start 140.97 118.745) (end 141.097 118.618) (width 1) (layer "F.Cu") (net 19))
 (segment (start 141.097 117.719) (end 142.113 116.703) (width 1) (layer "F.Cu") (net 19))
 (segment (start 140.97 118.745) (end 135.509 118.745) (width 1) (layer "F.Cu") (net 19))
 (segment (start 141.097 118.618) (end 141.097 117.719) (width 1) (layer "F.Cu") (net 19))
 (segment (start 133.096 121.158) (end 133.096 124.46) (width 1) (layer "F.Cu") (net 19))
 (segment (start 135.636 124.46) (end 135.636 122.682) (width 1) (layer "F.Cu") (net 20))
 (segment (start 142.367 121.285) (end 144.653 118.999) (width 1) (layer "F.Cu") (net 20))
 (segment (start 135.636 122.682) (end 137.033 121.285) (width 1) (layer "F.Cu") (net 20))
 (segment (start 137.033 121.285) (end 142.367 121.285) (width 1) (layer "F.Cu") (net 20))
 (segment (start 144.653 118.999) (end 144.653 116.703) (width 1) (layer "F.Cu") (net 20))
 (segment (start 182.15 127.381) (end 185.325 130.556) (width 1) (layer "F.Cu") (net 1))
 (segment (start 182.15 118.586) (end 182.15 127.381) (width 1) (layer "F.Cu") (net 1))
 (segment (start 192.334 108.077) (end 192.334 108.402) (width 1) (layer "F.Cu") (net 1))
 (segment (start 192.334 108.402) (end 182.15 118.586) (width 1) (layer "F.Cu") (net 1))
 (segment (start 150.876 142.24) (end 150.876 140.589) (width 1) (layer "F.Cu") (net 1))
 (segment (start 174.117 127.381) (end 182.15 127.381) (width 1) (layer "F.Cu") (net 1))
 (segment (start 158.623 132.842) (end 168.656 132.842) (width 1) (layer "F.Cu") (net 1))
 (segment (start 150.876 140.589) (end 158.623 132.842) (width 1) (layer "F.Cu") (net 1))
 (segment (start 168.656 132.842) (end 174.117 127.381) (width 1) (layer "F.Cu") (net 1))
 (segment (start 168.656 139.827) (end 171.704 136.779) (width 1) (layer "F.Cu") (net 8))
 (segment (start 198.12 136.779) (end 198.12 109.323) (width 1) (layer "F.Cu") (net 8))
 (segment (start 194.334 105.537) (end 192.334 105.537) (width 1) (layer "F.Cu") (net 8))
 (segment (start 168.656 142.24) (end 168.656 139.827) (width 1) (layer "F.Cu") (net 8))
 (segment (start 171.704 136.779) (end 198.12 136.779) (width 1) (layer "F.Cu") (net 8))
 (segment (start 198.12 109.323) (end 194.334 105.537) (width 1) (layer "F.Cu") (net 8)))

